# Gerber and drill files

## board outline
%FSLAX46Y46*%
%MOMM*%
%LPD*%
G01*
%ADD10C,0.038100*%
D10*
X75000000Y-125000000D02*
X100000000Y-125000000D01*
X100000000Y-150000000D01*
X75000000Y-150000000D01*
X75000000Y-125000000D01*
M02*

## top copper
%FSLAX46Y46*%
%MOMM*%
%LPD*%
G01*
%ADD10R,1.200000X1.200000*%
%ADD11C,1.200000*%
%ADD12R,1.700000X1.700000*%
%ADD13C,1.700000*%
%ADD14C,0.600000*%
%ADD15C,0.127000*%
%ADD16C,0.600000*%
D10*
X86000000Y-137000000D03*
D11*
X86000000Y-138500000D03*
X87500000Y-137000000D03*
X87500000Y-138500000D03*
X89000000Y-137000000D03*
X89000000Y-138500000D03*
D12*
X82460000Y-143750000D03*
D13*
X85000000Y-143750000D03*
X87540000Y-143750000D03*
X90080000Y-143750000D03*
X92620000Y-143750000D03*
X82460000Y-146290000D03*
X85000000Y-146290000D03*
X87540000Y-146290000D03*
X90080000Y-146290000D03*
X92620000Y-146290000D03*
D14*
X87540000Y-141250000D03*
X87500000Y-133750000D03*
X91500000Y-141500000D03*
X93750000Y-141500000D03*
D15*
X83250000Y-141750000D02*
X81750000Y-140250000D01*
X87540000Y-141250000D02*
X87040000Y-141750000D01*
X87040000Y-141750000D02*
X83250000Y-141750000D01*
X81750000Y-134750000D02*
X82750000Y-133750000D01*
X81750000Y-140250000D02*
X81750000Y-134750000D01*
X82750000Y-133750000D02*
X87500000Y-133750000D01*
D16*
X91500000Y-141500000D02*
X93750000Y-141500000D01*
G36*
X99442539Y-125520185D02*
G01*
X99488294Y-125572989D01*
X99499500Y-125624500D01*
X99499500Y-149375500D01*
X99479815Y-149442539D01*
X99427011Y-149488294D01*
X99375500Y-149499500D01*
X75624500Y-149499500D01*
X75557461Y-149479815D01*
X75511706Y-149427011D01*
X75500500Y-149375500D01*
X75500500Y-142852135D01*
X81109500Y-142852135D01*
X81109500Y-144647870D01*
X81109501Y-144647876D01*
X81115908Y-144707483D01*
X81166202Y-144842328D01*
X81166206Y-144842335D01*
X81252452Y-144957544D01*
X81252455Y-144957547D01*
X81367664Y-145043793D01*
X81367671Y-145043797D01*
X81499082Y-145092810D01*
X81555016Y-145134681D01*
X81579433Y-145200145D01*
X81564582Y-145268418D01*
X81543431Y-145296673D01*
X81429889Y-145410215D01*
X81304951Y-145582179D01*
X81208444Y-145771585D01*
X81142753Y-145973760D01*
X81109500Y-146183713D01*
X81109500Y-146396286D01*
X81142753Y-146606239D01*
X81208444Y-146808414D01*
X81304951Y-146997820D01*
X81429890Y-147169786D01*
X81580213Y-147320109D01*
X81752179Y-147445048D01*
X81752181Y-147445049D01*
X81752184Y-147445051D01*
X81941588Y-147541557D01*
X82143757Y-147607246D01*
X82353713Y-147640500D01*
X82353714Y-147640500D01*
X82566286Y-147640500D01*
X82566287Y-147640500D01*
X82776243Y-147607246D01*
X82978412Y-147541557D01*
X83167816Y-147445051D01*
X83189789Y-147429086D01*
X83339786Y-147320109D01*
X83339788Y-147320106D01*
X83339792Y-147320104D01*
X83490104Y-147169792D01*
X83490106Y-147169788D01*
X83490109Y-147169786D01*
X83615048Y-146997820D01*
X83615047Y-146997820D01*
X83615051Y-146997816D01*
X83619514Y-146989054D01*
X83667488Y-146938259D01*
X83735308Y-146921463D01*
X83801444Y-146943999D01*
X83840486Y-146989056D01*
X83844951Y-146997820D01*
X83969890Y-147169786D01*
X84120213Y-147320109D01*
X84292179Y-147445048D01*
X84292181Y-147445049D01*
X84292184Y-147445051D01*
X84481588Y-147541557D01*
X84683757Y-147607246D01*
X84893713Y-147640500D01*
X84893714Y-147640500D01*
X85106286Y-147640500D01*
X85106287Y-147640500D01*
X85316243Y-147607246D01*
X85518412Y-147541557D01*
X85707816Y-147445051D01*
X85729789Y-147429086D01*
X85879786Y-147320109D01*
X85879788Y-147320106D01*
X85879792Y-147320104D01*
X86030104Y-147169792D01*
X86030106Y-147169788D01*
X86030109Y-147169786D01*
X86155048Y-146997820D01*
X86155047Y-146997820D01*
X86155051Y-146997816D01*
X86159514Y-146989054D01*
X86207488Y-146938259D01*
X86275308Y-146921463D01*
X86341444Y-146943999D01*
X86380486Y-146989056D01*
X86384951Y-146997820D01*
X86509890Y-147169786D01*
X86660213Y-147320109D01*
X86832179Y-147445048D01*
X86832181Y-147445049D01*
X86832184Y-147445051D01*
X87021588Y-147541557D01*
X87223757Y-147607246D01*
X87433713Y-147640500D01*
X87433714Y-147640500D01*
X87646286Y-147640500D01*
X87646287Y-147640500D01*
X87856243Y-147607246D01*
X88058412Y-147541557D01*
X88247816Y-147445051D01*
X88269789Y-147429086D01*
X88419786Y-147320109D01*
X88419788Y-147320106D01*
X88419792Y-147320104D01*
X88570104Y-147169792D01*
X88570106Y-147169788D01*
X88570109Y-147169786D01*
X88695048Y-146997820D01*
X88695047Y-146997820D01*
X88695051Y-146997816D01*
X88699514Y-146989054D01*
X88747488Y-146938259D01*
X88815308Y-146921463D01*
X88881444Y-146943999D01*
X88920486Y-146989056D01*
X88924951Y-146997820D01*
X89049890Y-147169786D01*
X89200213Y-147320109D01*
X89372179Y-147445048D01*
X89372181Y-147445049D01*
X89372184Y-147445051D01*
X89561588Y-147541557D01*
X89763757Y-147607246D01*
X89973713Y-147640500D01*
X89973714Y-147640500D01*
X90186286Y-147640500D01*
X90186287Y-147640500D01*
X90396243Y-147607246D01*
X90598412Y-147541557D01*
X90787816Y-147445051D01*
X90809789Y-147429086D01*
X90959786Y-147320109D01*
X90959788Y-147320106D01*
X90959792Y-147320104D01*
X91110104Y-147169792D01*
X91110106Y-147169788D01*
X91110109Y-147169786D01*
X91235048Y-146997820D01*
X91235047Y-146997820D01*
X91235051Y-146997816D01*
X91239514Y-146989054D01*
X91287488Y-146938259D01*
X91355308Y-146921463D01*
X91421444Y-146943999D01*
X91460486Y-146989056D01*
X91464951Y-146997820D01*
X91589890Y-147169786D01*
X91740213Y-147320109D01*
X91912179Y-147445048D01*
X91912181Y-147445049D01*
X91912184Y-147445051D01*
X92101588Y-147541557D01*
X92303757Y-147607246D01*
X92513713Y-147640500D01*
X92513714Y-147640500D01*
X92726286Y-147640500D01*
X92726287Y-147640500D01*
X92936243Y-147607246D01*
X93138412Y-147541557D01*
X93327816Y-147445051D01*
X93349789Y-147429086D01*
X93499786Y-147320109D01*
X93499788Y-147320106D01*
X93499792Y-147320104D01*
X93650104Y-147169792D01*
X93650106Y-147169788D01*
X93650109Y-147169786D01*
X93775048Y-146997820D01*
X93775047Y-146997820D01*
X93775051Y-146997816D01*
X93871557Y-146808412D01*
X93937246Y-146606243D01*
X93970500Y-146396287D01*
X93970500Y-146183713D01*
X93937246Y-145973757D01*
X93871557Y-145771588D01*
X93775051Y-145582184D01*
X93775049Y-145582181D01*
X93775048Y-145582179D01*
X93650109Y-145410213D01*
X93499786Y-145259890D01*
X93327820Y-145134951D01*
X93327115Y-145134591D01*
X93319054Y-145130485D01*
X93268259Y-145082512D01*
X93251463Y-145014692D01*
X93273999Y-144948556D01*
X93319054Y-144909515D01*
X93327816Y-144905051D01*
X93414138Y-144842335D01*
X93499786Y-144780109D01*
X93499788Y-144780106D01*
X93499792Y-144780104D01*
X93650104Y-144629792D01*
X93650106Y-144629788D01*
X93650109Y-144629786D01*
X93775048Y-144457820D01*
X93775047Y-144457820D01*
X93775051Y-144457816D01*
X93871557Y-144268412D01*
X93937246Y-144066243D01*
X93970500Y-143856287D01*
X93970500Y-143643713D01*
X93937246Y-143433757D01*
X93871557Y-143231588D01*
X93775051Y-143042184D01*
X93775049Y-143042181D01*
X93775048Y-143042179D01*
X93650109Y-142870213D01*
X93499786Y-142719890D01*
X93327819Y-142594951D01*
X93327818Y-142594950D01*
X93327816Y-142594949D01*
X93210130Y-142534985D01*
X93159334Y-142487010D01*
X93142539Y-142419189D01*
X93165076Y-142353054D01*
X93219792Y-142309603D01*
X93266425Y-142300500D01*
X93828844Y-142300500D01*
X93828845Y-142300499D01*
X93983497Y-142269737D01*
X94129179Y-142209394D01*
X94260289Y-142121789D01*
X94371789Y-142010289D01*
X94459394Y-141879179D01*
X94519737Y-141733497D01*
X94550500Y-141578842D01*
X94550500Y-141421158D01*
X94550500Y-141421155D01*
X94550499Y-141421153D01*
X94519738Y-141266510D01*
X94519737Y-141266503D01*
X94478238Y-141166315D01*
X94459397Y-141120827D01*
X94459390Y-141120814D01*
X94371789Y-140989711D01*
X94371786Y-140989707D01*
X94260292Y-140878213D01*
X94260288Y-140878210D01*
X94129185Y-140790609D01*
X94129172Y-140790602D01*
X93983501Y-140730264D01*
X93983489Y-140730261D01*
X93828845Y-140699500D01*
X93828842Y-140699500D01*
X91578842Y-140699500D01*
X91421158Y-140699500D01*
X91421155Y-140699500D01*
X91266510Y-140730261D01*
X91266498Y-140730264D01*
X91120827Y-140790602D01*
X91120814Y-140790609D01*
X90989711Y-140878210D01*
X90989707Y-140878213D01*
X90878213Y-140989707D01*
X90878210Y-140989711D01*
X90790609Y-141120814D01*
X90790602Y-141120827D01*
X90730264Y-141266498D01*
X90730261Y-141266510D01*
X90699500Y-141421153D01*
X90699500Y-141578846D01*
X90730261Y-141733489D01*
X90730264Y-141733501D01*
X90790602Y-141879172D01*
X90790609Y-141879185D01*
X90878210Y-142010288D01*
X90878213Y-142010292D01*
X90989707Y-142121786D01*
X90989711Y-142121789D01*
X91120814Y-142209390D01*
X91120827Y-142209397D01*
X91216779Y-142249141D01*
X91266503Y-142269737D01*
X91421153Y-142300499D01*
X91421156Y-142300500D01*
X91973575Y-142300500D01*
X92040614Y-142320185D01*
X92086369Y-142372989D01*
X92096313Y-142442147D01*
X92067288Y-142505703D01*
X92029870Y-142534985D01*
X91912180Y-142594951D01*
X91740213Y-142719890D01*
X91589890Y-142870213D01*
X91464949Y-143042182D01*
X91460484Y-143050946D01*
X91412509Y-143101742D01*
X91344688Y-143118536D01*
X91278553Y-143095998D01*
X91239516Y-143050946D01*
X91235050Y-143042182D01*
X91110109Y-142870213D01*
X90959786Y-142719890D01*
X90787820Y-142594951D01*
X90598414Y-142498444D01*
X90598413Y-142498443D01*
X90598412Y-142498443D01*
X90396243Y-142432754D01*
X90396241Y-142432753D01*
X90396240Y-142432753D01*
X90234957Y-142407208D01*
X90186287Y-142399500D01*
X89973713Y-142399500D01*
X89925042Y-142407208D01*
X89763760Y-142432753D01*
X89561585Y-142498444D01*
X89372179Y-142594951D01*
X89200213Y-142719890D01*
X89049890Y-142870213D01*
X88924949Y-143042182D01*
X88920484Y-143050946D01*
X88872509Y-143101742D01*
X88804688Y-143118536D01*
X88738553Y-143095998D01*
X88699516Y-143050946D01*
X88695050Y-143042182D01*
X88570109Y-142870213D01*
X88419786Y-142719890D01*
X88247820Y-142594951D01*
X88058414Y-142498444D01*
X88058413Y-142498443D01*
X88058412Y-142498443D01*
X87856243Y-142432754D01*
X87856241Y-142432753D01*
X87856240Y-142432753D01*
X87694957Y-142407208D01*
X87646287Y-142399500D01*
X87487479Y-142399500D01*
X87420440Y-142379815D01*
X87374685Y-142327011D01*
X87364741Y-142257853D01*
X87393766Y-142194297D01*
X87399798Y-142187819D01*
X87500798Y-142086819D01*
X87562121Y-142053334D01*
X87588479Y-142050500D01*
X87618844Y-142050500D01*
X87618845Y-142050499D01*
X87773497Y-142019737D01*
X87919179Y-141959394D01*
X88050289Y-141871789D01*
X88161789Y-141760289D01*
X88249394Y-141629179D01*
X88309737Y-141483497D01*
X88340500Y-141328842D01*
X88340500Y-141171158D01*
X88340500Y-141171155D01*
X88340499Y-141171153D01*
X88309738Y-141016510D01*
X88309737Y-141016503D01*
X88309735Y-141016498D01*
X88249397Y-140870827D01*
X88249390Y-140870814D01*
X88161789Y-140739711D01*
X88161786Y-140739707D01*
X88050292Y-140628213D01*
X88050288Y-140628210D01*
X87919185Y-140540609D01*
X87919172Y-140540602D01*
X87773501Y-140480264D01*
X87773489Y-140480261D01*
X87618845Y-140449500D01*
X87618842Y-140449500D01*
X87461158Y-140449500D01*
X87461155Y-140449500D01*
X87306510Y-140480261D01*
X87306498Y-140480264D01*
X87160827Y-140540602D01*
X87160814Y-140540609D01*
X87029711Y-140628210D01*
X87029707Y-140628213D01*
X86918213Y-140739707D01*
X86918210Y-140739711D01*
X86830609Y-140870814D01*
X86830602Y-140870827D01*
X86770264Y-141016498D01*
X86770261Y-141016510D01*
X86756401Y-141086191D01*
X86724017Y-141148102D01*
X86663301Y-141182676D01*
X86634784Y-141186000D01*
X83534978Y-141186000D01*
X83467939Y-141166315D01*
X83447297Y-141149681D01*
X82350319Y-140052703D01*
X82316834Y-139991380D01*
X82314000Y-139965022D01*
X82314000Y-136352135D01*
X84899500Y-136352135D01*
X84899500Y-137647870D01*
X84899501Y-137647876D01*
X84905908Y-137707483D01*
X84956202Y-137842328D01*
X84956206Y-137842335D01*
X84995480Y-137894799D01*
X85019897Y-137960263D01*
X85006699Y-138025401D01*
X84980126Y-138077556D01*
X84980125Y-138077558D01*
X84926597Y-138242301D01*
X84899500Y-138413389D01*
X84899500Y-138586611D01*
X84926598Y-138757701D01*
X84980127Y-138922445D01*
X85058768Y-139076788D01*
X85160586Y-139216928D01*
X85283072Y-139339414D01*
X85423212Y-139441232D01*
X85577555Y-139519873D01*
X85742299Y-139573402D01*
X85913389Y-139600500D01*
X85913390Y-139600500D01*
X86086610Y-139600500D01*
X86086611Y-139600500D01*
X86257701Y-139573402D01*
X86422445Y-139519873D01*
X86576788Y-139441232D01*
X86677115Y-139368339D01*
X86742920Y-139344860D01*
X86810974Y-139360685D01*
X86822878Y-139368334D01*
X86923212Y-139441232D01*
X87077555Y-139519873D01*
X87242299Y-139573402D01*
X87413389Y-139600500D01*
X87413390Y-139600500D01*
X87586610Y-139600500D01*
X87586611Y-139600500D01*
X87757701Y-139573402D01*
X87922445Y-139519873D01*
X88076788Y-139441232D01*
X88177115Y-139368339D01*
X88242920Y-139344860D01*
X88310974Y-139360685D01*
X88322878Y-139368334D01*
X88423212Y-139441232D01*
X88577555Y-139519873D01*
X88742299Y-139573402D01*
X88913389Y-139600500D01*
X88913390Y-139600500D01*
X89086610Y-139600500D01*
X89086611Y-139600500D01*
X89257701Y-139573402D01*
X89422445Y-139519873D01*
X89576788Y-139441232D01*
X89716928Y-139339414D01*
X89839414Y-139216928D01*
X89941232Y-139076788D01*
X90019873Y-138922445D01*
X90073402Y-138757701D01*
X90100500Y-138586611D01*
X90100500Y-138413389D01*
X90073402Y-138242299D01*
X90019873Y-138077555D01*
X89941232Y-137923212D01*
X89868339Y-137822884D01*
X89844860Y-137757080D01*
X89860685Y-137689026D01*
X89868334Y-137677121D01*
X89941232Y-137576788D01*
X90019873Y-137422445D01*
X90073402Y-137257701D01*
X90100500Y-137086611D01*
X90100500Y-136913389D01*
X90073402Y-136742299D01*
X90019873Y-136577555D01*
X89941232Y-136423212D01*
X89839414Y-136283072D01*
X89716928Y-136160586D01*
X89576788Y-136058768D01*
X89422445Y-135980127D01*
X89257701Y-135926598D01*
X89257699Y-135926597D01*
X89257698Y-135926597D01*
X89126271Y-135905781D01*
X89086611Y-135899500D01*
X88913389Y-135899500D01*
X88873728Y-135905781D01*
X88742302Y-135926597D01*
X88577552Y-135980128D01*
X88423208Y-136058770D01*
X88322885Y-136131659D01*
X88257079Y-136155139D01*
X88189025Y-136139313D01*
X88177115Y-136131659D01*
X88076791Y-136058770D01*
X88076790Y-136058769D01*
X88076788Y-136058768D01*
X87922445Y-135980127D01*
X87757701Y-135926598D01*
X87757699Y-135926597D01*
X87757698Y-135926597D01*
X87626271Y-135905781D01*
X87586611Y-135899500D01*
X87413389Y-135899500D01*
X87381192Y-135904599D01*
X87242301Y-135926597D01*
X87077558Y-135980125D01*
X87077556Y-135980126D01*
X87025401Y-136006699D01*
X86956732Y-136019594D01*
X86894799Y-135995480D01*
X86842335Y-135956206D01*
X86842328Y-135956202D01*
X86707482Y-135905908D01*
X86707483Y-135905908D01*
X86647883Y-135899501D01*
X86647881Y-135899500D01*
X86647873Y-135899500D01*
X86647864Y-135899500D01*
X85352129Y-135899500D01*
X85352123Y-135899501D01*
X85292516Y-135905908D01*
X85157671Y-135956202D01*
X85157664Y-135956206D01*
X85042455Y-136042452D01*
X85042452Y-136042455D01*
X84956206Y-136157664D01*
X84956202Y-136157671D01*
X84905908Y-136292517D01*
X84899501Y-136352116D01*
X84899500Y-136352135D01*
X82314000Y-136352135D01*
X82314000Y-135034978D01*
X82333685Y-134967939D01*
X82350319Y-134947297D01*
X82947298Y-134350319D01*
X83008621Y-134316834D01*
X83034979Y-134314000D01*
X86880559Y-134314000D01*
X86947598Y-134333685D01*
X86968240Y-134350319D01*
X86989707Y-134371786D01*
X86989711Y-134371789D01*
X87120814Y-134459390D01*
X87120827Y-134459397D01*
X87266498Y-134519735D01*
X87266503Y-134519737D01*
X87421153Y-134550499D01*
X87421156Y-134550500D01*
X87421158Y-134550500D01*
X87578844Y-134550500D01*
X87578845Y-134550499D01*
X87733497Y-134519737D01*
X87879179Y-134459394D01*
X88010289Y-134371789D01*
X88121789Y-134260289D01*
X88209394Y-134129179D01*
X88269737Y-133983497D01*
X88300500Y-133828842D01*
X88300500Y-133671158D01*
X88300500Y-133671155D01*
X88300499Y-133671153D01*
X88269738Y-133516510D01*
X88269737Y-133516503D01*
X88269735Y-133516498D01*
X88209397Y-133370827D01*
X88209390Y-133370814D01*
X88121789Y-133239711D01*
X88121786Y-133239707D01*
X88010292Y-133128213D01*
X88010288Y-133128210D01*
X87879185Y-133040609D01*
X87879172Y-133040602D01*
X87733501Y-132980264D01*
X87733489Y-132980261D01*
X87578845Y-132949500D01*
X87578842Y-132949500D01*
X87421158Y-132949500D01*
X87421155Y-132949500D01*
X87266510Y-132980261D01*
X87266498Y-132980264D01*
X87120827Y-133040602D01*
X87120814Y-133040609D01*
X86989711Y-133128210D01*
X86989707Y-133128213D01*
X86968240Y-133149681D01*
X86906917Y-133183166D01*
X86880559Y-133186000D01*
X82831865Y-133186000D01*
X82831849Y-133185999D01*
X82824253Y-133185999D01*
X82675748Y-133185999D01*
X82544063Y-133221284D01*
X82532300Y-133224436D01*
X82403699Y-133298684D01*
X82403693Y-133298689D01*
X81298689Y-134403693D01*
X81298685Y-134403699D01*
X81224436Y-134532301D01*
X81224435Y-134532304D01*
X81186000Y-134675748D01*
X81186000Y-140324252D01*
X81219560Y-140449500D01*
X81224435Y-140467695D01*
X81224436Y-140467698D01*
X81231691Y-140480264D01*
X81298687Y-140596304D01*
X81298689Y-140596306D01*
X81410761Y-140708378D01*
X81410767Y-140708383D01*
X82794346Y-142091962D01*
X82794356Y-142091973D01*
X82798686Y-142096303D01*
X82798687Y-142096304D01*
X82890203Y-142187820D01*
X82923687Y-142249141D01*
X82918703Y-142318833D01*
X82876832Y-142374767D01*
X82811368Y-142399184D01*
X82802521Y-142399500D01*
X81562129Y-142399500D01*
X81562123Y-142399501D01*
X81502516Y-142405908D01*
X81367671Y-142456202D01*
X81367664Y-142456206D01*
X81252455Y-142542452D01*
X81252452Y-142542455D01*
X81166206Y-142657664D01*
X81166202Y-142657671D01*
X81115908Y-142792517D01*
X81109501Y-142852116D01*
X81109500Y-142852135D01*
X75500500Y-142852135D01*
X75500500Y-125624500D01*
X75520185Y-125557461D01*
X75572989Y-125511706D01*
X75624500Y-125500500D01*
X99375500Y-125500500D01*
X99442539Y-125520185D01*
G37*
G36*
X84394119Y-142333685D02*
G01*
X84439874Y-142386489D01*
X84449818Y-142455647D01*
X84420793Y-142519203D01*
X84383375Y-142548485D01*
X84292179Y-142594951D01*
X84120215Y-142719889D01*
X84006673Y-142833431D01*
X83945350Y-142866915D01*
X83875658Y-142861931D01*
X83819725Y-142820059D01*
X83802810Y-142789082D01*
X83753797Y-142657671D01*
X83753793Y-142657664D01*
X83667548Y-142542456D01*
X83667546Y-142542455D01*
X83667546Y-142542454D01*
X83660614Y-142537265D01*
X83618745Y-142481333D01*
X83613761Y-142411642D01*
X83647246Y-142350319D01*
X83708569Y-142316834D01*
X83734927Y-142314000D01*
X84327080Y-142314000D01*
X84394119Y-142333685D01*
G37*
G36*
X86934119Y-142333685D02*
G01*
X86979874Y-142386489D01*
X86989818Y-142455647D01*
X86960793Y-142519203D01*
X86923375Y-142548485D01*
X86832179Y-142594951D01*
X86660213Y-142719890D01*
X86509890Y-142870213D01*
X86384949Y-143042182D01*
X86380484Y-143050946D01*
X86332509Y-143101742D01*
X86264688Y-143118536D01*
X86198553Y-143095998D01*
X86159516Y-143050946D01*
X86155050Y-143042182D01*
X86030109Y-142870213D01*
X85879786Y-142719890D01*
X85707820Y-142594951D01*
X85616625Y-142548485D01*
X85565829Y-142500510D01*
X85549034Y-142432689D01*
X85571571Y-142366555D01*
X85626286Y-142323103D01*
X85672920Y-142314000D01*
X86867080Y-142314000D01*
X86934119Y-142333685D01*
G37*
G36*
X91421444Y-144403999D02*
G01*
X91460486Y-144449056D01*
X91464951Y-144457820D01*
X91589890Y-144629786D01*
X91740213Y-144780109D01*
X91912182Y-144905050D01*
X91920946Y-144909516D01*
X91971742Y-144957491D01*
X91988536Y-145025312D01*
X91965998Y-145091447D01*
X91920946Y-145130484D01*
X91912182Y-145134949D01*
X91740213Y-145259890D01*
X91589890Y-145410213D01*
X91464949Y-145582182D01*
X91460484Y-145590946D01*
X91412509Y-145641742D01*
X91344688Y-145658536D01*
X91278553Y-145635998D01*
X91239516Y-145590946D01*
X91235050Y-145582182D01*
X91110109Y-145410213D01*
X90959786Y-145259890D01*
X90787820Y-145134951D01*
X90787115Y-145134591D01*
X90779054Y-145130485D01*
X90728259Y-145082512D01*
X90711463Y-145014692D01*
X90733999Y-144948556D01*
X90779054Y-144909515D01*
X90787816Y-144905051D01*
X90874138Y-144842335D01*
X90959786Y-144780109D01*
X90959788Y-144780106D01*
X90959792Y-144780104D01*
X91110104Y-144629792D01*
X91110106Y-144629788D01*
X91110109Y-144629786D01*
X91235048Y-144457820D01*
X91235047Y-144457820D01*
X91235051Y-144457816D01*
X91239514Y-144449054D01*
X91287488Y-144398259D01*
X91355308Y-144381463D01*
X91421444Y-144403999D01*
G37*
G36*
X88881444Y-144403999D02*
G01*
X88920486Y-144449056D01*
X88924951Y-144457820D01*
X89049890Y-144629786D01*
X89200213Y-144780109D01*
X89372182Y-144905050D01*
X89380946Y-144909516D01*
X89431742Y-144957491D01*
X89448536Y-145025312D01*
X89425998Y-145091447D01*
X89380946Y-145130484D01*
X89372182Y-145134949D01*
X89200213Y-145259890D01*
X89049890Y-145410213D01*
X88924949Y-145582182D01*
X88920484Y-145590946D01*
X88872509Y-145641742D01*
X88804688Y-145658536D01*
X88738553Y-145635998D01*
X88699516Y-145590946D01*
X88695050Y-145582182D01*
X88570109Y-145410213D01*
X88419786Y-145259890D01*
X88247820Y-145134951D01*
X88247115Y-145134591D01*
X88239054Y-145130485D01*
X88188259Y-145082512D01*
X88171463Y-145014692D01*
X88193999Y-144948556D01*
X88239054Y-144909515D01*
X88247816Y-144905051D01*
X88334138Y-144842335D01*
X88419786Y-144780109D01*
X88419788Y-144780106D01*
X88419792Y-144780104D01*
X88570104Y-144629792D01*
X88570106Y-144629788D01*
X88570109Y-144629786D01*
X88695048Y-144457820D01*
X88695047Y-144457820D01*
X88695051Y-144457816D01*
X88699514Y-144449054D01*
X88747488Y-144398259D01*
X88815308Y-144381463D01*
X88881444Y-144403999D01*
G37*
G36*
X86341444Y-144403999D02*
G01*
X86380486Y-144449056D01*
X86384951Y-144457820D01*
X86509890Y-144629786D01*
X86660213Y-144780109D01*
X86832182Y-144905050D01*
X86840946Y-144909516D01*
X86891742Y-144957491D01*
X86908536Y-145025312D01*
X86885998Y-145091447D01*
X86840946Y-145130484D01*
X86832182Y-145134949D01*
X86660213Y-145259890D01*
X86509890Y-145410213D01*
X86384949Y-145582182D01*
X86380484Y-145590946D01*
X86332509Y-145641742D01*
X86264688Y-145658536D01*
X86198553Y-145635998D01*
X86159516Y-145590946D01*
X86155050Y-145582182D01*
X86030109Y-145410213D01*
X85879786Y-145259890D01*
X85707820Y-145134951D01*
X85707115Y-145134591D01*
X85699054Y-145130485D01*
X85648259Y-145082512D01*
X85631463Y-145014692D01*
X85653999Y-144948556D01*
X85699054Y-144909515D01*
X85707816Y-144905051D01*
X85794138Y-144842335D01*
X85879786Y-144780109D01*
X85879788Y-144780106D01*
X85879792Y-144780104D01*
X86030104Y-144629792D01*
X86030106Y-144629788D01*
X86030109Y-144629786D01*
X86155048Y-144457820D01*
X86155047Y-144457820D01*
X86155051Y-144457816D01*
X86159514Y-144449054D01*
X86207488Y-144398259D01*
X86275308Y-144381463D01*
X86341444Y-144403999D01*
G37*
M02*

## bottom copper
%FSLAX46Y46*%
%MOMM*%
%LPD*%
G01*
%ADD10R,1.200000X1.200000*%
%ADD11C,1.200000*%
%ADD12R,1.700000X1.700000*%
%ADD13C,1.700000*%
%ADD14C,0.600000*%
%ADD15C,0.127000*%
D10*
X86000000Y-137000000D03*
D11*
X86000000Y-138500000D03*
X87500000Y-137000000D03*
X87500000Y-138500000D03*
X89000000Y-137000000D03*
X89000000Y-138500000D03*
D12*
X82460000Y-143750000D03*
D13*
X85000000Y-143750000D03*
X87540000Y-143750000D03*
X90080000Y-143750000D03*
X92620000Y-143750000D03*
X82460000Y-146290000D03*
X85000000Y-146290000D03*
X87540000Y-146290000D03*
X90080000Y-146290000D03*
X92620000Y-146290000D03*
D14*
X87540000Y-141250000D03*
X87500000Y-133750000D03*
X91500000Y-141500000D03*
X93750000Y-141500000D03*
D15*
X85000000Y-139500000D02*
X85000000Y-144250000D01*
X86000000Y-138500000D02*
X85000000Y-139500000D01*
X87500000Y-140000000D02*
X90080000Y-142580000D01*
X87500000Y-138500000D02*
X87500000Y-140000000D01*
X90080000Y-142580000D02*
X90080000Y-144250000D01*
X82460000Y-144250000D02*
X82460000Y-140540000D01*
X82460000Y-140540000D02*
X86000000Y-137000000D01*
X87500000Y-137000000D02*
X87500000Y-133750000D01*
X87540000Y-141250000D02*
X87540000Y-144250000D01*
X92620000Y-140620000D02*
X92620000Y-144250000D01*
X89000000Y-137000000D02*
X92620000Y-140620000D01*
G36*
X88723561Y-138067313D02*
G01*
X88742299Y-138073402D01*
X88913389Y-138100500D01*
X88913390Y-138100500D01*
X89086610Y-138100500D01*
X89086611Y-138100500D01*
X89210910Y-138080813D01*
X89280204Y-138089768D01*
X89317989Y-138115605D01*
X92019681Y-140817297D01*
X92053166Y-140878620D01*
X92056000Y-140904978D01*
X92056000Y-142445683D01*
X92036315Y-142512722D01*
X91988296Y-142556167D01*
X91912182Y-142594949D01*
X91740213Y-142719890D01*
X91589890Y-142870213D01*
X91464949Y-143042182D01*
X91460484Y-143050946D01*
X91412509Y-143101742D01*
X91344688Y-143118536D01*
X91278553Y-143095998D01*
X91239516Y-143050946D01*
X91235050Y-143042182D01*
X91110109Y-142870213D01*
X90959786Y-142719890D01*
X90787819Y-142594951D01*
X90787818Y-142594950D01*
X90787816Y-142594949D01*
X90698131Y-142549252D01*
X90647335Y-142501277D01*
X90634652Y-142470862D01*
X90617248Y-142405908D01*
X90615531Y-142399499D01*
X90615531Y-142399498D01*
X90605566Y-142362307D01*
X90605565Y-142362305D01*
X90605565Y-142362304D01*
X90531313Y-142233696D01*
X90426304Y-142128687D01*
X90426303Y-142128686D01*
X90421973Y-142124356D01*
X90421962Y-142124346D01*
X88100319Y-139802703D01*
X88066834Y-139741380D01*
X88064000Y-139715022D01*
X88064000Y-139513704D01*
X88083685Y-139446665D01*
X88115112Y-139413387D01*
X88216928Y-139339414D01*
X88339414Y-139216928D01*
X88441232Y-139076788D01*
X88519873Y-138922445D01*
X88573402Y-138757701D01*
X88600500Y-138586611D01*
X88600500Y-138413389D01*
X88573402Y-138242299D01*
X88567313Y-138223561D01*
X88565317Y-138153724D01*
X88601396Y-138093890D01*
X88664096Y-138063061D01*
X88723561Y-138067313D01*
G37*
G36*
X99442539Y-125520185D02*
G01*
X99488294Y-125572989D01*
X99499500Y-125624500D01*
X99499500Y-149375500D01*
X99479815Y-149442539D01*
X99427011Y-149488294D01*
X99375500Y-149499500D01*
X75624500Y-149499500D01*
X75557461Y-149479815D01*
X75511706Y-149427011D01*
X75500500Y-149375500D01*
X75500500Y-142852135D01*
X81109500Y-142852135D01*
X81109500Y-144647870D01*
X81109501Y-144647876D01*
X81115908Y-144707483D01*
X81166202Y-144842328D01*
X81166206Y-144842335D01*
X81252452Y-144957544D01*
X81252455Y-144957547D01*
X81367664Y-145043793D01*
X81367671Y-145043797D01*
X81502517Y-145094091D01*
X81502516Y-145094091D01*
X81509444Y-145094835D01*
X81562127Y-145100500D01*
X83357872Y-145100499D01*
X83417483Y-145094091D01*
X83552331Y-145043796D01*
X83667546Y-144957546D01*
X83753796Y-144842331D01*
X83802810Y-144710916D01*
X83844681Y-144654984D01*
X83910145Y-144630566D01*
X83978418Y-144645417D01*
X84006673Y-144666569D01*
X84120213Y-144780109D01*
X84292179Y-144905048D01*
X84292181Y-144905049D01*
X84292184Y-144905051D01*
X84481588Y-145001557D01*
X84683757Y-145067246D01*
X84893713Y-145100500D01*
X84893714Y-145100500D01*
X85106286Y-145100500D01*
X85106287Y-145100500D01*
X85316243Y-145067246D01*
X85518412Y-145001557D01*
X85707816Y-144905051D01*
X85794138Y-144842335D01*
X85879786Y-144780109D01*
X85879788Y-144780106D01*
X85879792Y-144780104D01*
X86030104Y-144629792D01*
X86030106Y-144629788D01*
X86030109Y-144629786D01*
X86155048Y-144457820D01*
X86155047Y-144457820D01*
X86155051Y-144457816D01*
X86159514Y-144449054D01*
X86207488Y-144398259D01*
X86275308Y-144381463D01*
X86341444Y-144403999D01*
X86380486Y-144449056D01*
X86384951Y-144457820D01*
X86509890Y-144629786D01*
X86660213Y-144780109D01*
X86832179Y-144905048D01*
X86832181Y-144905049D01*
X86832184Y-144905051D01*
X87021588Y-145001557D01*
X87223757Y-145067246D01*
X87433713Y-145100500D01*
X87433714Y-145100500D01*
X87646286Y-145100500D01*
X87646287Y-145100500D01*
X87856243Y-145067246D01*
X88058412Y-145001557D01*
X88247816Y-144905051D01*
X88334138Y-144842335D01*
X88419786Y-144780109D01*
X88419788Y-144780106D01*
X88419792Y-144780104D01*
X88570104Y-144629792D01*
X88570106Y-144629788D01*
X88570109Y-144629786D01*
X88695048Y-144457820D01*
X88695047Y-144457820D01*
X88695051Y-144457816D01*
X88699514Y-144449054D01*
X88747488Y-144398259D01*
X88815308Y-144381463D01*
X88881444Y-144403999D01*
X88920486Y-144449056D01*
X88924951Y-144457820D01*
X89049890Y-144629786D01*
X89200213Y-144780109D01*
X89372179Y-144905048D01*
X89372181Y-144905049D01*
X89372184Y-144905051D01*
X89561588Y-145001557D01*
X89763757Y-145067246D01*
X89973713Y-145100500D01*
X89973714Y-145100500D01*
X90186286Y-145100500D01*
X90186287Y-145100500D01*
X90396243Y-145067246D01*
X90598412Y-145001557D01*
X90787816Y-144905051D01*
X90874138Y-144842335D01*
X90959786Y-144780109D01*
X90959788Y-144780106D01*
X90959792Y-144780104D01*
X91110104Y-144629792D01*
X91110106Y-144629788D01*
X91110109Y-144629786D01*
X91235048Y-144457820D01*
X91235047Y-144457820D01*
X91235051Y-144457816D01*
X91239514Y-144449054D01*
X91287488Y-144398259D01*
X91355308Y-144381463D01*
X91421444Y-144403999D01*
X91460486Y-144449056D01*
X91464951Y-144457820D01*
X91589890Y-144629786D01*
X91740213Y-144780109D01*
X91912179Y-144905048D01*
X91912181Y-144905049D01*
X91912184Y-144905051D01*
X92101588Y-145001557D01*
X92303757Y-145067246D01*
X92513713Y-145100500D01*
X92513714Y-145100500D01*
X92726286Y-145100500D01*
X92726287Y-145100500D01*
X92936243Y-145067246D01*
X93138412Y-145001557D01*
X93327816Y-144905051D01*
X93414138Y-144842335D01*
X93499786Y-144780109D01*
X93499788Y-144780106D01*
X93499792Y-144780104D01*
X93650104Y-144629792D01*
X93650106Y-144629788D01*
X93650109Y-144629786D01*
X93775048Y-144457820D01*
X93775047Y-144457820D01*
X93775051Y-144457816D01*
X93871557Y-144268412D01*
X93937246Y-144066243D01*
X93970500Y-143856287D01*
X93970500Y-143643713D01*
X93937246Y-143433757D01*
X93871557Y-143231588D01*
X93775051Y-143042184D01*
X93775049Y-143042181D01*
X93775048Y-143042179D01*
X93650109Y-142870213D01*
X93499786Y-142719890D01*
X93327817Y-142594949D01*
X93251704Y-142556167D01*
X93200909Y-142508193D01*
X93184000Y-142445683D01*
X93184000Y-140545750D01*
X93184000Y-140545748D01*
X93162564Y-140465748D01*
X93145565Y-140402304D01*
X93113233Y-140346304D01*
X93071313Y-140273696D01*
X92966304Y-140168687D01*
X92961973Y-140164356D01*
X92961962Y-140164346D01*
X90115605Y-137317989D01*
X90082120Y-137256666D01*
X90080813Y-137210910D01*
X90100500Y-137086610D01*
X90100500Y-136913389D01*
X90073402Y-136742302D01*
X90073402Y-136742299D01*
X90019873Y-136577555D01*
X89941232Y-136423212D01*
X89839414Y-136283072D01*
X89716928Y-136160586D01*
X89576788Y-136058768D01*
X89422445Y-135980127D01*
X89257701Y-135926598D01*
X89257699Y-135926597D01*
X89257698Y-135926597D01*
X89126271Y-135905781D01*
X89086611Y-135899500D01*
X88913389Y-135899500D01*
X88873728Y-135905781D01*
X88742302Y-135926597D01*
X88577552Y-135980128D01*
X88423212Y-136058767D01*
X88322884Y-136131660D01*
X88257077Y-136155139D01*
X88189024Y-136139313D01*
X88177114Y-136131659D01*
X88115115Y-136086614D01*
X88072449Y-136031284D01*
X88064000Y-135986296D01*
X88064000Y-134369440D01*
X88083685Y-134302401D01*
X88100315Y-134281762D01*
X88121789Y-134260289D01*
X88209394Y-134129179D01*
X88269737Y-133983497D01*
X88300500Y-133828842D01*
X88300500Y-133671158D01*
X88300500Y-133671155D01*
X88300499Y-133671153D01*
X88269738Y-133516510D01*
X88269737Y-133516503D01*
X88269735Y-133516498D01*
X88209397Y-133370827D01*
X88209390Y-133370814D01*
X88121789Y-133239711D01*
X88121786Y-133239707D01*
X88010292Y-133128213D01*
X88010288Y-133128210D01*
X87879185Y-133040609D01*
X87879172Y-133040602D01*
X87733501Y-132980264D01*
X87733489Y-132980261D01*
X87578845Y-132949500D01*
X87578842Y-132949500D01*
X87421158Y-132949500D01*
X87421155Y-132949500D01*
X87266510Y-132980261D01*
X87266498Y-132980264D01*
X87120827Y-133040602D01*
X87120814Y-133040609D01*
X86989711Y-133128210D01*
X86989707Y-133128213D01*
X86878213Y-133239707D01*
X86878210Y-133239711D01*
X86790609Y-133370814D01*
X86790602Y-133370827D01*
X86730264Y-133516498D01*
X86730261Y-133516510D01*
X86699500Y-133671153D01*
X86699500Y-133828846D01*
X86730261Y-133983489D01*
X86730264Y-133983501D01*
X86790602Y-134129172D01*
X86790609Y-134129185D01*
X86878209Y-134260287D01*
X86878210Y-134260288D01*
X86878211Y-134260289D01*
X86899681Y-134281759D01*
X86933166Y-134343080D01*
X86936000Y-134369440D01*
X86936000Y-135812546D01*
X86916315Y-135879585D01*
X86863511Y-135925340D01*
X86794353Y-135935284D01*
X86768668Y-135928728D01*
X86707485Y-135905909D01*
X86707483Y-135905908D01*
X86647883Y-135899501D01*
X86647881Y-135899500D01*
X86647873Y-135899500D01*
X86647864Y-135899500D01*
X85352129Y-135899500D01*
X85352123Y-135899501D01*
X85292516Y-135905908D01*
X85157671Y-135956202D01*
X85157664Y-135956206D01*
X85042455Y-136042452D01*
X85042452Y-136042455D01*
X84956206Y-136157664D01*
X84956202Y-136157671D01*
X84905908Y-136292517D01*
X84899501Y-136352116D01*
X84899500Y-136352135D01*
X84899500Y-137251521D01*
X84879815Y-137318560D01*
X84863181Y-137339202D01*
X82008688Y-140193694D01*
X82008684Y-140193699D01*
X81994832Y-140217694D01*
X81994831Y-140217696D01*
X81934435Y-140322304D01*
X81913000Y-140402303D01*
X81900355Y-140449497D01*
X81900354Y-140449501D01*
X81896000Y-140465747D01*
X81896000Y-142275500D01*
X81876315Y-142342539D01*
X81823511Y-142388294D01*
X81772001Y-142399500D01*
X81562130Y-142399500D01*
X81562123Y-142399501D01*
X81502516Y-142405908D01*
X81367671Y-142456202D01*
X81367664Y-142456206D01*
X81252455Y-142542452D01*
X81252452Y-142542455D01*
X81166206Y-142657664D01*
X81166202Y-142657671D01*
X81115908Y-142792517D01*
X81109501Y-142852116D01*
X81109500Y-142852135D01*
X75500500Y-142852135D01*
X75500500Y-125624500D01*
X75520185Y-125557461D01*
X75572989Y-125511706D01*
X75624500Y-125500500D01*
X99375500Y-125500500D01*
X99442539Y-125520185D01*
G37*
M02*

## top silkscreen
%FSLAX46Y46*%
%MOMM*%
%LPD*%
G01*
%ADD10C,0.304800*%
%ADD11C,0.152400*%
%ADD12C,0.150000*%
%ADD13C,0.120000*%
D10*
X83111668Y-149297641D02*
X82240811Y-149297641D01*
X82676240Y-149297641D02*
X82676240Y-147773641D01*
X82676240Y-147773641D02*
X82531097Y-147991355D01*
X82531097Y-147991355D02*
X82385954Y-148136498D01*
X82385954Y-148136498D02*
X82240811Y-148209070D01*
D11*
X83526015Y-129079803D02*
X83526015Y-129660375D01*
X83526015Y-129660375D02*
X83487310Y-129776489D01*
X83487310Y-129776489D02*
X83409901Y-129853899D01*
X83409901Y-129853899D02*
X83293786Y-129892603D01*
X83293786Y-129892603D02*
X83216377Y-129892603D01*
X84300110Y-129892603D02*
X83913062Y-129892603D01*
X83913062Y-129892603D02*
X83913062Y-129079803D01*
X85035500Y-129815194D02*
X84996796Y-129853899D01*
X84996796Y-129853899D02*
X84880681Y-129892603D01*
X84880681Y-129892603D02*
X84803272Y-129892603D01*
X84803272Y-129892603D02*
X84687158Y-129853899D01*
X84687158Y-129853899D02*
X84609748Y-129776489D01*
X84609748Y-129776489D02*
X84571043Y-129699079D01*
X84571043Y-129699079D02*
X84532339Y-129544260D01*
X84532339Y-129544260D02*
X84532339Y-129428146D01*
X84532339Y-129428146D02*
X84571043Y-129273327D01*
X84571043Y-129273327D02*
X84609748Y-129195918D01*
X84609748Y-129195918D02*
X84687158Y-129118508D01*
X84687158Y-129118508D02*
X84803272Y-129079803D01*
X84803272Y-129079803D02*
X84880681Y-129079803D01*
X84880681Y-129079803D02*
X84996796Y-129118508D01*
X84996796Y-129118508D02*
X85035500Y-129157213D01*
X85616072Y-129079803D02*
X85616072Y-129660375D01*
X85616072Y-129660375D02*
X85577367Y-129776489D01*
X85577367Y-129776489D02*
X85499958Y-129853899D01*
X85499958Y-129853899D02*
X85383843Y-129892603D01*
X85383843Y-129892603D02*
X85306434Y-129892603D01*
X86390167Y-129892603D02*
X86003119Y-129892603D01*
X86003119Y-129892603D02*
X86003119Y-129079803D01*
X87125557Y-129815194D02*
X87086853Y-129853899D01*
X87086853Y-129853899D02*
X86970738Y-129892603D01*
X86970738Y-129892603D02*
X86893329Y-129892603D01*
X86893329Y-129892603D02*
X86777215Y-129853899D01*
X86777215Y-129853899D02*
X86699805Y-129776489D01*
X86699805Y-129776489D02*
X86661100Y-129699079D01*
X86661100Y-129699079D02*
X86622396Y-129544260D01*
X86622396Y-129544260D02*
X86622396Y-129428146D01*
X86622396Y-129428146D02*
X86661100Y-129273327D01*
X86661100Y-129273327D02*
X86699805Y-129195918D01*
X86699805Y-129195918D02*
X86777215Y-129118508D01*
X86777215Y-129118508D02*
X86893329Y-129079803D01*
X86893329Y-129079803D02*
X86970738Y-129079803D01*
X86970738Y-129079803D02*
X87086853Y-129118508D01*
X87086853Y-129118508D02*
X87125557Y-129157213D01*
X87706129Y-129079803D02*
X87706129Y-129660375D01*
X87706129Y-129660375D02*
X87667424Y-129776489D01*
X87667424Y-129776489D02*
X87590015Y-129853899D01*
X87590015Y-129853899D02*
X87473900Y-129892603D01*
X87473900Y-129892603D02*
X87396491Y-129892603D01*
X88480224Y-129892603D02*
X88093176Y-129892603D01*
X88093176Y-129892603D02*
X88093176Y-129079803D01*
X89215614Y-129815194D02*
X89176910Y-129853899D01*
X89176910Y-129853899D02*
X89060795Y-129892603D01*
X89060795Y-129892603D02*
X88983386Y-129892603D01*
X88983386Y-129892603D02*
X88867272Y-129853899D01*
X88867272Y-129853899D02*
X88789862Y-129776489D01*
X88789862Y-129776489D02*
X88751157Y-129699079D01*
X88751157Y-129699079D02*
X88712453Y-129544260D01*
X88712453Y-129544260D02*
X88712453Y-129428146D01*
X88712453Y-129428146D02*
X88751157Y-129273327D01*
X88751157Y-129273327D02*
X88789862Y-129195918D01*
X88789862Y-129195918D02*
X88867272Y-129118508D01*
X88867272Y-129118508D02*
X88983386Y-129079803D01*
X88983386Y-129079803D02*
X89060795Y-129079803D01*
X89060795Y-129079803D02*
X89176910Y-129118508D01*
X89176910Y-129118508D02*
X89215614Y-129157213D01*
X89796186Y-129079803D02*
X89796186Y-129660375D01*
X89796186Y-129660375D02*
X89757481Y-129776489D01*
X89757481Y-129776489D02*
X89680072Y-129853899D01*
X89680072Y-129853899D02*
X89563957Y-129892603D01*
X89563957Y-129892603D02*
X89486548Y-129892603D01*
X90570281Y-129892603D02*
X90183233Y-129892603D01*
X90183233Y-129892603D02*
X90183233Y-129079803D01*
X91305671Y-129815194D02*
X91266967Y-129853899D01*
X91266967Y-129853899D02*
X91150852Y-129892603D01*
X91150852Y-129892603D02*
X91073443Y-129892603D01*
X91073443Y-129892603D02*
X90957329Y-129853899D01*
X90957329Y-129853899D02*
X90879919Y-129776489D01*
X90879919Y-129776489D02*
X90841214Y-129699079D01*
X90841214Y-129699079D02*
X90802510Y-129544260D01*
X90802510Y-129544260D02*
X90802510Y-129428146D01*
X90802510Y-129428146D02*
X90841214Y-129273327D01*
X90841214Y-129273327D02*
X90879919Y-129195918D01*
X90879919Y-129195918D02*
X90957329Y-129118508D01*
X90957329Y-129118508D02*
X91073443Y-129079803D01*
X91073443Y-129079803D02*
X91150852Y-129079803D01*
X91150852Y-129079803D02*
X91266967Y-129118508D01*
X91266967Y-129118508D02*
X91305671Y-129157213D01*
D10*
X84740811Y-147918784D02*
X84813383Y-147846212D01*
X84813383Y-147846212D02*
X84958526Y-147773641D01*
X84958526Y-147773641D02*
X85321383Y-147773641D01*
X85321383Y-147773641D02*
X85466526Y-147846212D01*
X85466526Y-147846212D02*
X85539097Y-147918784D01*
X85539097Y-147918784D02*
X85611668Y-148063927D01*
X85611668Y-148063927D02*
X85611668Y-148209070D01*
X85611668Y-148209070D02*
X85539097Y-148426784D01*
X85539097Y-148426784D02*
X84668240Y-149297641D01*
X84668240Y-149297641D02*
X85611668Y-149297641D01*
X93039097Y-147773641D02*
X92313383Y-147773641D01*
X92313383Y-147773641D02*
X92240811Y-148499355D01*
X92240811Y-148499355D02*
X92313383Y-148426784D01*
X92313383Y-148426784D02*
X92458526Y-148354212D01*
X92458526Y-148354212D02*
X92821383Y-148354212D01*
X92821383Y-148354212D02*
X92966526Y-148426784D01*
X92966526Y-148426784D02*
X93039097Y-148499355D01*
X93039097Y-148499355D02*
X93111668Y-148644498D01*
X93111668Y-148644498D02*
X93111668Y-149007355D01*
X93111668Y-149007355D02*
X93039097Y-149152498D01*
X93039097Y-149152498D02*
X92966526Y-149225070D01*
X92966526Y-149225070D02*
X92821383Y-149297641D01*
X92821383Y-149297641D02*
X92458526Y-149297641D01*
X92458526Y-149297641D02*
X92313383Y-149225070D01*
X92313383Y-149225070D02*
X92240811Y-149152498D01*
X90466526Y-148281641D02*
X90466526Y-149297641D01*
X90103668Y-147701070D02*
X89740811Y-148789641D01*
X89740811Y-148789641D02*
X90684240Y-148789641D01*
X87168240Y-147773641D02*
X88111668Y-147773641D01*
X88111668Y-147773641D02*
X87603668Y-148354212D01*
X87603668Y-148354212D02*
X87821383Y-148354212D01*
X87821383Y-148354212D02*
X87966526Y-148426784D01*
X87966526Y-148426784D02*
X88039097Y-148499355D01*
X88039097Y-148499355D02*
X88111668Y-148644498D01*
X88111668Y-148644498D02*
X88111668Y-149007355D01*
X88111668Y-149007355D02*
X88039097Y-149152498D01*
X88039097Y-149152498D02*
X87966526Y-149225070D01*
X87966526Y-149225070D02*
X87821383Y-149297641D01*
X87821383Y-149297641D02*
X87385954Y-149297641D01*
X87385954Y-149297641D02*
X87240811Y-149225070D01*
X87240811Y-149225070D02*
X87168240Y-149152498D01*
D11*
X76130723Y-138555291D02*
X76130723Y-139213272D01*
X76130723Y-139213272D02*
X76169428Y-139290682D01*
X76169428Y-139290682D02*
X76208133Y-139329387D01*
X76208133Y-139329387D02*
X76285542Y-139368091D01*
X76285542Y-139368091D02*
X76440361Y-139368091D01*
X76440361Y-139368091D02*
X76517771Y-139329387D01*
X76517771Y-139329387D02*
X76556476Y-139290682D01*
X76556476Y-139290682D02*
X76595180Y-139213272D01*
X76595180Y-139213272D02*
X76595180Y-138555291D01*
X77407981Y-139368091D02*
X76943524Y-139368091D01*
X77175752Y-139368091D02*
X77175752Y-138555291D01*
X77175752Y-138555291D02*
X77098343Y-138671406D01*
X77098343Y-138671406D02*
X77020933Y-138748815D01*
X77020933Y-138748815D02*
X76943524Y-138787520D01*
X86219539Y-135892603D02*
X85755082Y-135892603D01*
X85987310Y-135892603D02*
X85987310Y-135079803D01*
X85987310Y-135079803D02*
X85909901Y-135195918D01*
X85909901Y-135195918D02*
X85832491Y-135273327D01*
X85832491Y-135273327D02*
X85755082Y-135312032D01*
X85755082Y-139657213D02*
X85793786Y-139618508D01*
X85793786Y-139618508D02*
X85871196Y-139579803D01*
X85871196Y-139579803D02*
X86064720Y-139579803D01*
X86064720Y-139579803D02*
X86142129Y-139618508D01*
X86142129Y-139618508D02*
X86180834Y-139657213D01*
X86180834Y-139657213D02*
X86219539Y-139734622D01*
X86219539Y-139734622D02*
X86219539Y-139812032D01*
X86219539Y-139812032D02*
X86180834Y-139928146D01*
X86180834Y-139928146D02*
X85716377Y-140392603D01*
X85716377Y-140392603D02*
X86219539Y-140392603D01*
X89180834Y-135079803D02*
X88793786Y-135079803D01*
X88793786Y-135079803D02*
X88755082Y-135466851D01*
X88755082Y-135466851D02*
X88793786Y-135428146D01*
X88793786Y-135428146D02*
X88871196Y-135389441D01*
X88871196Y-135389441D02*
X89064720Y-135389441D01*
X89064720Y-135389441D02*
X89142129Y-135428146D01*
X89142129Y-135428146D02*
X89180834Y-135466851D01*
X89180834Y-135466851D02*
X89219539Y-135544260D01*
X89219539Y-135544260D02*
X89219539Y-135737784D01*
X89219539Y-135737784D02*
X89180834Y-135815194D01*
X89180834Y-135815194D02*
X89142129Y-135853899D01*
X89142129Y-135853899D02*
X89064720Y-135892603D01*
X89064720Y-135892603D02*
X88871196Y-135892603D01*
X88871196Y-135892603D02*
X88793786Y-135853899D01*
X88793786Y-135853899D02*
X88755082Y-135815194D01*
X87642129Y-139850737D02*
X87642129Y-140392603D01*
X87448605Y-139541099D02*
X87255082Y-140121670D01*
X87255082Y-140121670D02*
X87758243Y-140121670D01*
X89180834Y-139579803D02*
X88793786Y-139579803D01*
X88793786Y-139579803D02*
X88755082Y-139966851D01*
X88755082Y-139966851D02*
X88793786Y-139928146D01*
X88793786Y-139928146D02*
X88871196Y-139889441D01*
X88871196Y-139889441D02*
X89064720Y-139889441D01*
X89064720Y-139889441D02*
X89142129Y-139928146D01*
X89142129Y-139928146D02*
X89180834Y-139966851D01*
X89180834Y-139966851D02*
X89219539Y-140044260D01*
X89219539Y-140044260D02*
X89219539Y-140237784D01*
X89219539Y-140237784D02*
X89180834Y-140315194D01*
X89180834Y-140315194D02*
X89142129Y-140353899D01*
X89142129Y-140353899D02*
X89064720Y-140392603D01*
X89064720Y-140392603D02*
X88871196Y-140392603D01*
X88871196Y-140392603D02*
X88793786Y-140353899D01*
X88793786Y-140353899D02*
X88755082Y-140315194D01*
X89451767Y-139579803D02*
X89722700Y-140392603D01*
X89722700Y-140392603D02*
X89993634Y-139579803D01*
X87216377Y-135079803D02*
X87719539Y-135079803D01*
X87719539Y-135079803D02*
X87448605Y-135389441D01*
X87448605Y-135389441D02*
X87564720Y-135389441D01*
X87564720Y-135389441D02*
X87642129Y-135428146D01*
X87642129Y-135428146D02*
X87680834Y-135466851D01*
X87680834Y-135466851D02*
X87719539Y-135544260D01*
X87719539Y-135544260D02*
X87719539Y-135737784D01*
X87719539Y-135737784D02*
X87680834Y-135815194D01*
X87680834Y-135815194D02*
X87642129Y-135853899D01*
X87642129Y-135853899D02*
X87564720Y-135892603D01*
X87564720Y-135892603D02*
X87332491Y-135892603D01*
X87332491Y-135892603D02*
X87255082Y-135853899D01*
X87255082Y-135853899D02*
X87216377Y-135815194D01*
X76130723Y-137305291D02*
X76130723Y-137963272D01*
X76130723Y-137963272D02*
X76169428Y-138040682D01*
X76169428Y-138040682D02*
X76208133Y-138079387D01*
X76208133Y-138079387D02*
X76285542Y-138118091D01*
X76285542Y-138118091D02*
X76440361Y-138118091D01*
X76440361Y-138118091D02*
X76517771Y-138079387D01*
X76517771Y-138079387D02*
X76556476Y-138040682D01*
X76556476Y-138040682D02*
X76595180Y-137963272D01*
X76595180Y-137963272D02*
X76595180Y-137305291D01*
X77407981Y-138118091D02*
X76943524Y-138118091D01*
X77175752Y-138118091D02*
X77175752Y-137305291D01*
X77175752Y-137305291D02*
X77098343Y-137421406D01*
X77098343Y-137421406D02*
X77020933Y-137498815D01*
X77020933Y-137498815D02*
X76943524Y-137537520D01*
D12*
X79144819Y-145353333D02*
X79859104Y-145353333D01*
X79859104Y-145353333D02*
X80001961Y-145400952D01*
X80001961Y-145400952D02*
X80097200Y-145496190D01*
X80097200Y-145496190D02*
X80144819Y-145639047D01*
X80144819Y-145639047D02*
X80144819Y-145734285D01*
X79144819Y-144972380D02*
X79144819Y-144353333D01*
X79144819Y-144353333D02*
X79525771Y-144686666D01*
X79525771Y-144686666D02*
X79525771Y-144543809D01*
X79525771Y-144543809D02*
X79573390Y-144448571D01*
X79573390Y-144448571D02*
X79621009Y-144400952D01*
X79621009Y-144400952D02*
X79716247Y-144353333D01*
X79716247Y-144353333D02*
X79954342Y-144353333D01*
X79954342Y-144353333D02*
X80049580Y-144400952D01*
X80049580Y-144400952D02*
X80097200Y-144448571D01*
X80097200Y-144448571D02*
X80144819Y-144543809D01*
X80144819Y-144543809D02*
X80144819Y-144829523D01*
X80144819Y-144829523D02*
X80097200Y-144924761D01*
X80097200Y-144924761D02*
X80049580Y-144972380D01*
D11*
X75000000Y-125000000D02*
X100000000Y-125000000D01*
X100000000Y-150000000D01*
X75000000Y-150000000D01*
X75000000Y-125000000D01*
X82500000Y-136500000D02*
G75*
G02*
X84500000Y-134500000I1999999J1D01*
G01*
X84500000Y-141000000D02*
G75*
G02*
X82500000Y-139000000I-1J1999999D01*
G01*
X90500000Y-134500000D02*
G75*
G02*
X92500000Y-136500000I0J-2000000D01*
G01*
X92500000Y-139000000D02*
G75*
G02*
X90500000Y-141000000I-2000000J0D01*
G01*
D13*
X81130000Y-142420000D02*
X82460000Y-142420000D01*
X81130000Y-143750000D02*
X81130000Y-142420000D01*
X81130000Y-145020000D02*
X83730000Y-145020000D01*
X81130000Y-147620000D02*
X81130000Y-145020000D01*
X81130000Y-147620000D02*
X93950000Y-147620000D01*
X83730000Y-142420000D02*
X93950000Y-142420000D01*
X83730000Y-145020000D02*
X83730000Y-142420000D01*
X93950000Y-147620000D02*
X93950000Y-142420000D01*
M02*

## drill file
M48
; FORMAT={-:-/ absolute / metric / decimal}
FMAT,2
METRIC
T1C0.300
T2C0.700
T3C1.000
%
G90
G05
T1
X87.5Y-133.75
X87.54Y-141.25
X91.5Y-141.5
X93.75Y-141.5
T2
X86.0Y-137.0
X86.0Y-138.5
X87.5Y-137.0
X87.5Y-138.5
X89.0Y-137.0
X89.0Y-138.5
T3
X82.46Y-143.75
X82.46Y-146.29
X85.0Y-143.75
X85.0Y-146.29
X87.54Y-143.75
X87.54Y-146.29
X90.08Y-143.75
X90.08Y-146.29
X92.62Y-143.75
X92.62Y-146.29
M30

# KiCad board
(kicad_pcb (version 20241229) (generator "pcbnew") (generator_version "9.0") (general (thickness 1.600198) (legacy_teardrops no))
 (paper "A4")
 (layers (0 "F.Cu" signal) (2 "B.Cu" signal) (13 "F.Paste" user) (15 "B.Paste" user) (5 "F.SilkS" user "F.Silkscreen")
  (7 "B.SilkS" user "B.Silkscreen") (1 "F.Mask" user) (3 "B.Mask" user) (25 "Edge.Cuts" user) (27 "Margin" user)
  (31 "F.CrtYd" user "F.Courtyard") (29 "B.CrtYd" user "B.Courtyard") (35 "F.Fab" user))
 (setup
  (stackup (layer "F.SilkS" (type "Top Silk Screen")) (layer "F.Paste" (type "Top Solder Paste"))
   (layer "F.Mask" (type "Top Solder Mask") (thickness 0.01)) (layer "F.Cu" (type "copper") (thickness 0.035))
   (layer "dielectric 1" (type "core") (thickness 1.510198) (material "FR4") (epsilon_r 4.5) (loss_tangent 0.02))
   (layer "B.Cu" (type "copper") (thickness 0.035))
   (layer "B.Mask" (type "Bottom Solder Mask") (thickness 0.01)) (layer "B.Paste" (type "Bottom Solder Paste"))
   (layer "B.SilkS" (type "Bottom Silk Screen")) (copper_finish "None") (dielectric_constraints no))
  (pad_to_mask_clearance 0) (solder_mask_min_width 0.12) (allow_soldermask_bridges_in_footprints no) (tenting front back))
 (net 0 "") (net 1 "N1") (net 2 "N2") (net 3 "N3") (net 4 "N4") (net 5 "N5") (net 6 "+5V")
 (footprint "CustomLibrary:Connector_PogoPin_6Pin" (layer "F.Cu") (at 87.5 138)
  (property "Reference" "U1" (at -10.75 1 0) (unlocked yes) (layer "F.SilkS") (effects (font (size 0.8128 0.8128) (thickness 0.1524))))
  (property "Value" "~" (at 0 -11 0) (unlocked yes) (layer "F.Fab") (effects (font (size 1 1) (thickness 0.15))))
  (fp_rect (start -12.5 -13) (end 12.5 12) (stroke (width 0.1524) (type default)) (fill no) (layer "F.SilkS"))
  (fp_arc (start -5 -1.5) (mid -4.414214 -2.914214) (end -3 -3.5) (stroke (width 0.1524) (type default)) (layer "F.SilkS"))
  (fp_arc (start -3 3) (mid -4.414214 2.414214) (end -5 1) (stroke (width 0.1524) (type default)) (layer "F.SilkS"))
  (fp_arc (start 3 -3.5) (mid 4.414214 -2.914214) (end 5 -1.5) (stroke (width 0.1524) (type default)) (layer "F.SilkS"))
  (fp_arc (start 5 1) (mid 4.414214 2.414214) (end 3 3) (stroke (width 0.1524) (type default)) (layer "F.SilkS"))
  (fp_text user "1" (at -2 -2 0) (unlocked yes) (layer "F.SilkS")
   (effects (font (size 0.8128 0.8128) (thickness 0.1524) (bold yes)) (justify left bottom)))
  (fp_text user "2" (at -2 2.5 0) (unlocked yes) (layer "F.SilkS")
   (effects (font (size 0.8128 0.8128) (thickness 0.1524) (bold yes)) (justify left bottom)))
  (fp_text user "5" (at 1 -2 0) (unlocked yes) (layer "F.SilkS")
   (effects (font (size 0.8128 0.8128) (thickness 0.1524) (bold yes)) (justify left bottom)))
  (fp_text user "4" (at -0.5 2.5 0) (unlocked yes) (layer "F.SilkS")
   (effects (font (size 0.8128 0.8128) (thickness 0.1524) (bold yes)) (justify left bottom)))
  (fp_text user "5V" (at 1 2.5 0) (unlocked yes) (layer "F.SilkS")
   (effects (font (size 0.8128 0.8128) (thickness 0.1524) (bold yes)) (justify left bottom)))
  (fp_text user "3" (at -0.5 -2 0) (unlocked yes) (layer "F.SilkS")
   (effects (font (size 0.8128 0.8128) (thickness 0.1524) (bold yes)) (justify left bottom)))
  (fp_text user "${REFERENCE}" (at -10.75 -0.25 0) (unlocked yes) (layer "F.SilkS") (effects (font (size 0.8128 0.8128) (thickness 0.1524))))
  (pad "1" thru_hole rect (at -1.5 -1) (size 1.2 1.2) (drill 0.7) (layers "*.Cu" "*.Mask") (remove_unused_layers no) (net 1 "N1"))
  (pad "2" thru_hole circle (at -1.5 0.5) (size 1.2 1.2) (drill 0.7) (layers "*.Cu" "*.Mask") (remove_unused_layers no) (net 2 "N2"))
  (pad "3" thru_hole circle (at 0 -1) (size 1.2 1.2) (drill 0.7) (layers "*.Cu" "*.Mask") (remove_unused_layers no) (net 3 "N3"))
  (pad "4" thru_hole circle (at 0 0.5) (size 1.2 1.2) (drill 0.7) (layers "*.Cu" "*.Mask") (remove_unused_layers no) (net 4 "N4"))
  (pad "5" thru_hole circle (at 1.5 -1) (size 1.2 1.2) (drill 0.7) (layers "*.Cu" "*.Mask") (remove_unused_layers no) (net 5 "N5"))
  (pad "6" thru_hole circle (at 1.5 0.5) (size 1.2 1.2) (drill 0.7) (layers "*.Cu" "*.Mask") (remove_unused_layers no) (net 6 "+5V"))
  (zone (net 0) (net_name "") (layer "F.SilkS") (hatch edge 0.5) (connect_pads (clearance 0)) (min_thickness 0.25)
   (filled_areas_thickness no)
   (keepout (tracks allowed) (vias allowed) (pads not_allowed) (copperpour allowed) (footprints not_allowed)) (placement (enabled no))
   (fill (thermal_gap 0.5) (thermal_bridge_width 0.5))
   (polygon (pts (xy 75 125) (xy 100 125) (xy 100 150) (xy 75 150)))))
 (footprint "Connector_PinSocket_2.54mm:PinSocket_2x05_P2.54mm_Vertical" (layer "F.Cu") (at 82.46 143.75 90)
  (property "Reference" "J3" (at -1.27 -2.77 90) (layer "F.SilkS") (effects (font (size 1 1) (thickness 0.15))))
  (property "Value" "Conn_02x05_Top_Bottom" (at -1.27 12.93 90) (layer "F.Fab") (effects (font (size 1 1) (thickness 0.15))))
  (fp_line (start 1.33 -1.33) (end 1.33 0) (stroke (width 0.12) (type solid)) (layer "F.SilkS"))
  (fp_line (start 0 -1.33) (end 1.33 -1.33) (stroke (width 0.12) (type solid)) (layer "F.SilkS"))
  (fp_line (start -1.27 -1.33) (end -1.27 1.27) (stroke (width 0.12) (type solid)) (layer "F.SilkS"))
  (fp_line (start -3.87 -1.33) (end -1.27 -1.33) (stroke (width 0.12) (type solid)) (layer "F.SilkS"))
  (fp_line (start -3.87 -1.33) (end -3.87 11.49) (stroke (width 0.12) (type solid)) (layer "F.SilkS"))
  (fp_line (start 1.33 1.27) (end 1.33 11.49) (stroke (width 0.12) (type solid)) (layer "F.SilkS"))
  (fp_line (start -1.27 1.27) (end 1.33 1.27) (stroke (width 0.12) (type solid)) (layer "F.SilkS"))
  (fp_line (start -3.87 11.49) (end 1.33 11.49) (stroke (width 0.12) (type solid)) (layer "F.SilkS"))
  (pad "1" thru_hole rect (at 0 0 90) (size 1.7 1.7) (drill 1) (layers "*.Cu" "*.Mask") (remove_unused_layers no) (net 1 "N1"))
  (pad "2" thru_hole circle (at 0 2.54 90) (size 1.7 1.7) (drill 1) (layers "*.Cu" "*.Mask") (remove_unused_layers no) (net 2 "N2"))
  (pad "3" thru_hole circle (at 0 5.08 90) (size 1.7 1.7) (drill 1) (layers "*.Cu" "*.Mask") (remove_unused_layers no) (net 3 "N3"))
  (pad "4" thru_hole circle (at 0 7.62 90) (size 1.7 1.7) (drill 1) (layers "*.Cu" "*.Mask" "B.Adhes") (remove_unused_layers no)
   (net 4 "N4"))
  (pad "5" thru_hole circle (at 0 10.16 90) (size 1.7 1.7) (drill 1) (layers "*.Cu" "*.Mask") (remove_unused_layers no) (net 5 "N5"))
  (pad "6" thru_hole circle (at -2.54 0 90) (size 1.7 1.7) (drill 1) (layers "*.Cu" "*.Mask") (remove_unused_layers no) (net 6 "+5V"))
  (pad "7" thru_hole circle (at -2.54 2.54 90) (size 1.7 1.7) (drill 1) (layers "*.Cu" "*.Mask") (remove_unused_layers no) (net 6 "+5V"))
  (pad "8" thru_hole circle (at -2.54 5.08 90) (size 1.7 1.7) (drill 1) (layers "*.Cu" "*.Mask") (remove_unused_layers no) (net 6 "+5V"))
  (pad "9" thru_hole circle (at -2.54 7.62 90) (size 1.7 1.7) (drill 1) (layers "*.Cu" "*.Mask") (remove_unused_layers no) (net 6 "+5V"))
  (pad "10" thru_hole circle (at -2.54 10.16 90) (size 1.7 1.7) (drill 1) (layers "*.Cu" "*.Mask") (remove_unused_layers no) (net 6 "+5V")))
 (gr_rect (start 75 125) (end 100 150) (stroke (width 0.0381) (type solid)) (fill no) (layer "Edge.Cuts"))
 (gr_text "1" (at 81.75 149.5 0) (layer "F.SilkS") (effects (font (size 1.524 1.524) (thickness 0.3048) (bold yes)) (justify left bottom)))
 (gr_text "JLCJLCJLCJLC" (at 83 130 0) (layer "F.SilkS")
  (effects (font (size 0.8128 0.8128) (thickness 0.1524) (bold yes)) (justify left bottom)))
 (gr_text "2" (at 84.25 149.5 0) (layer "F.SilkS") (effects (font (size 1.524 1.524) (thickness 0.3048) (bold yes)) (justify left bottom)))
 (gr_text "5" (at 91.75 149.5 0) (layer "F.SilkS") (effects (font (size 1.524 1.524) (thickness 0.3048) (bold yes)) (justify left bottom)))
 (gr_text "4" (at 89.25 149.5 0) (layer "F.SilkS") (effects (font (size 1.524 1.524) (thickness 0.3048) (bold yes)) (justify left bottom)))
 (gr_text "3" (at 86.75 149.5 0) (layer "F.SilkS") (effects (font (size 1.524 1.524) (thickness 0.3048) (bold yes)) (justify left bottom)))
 (segment (start 85 139.5) (end 85 144.25) (width 0.127) (layer "B.Cu") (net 2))
 (segment (start 86 138.5) (end 85 139.5) (width 0.127) (layer "B.Cu") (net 2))
 (segment (start 87.5 140) (end 90.08 142.58) (width 0.127) (layer "B.Cu") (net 4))
 (segment (start 87.5 138.5) (end 87.5 140) (width 0.127) (layer "B.Cu") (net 4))
 (segment (start 90.08 142.58) (end 90.08 144.25) (width 0.127) (layer "B.Cu") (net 4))
 (segment (start 82.46 144.25) (end 82.46 140.54) (width 0.127) (layer "B.Cu") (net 1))
 (segment (start 82.46 140.54) (end 86 137) (width 0.127) (layer "B.Cu") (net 1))
 (segment (start 83.25 141.75) (end 81.75 140.25) (width 0.127) (layer "F.Cu") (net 3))
 (segment (start 87.54 141.25) (end 87.04 141.75) (width 0.127) (layer "F.Cu") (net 3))
 (segment (start 87.04 141.75) (end 83.25 141.75) (width 0.127) (layer "F.Cu") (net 3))
 (segment (start 81.75 134.75) (end 82.75 133.75) (width 0.127) (layer "F.Cu") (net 3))
 (segment (start 81.75 140.25) (end 81.75 134.75) (width 0.127) (layer "F.Cu") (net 3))
 (segment (start 82.75 133.75) (end 87.5 133.75) (width 0.127) (layer "F.Cu") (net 3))
 (via (at 87.54 141.25) (size 0.6) (drill 0.3) (layers "F.Cu" "B.Cu") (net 3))
 (via (at 87.5 133.75) (size 0.6) (drill 0.3) (layers "F.Cu" "B.Cu") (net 3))
 (segment (start 87.5 137) (end 87.5 133.75) (width 0.127) (layer "B.Cu") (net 3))
 (segment (start 87.54 141.25) (end 87.54 144.25) (width 0.127) (layer "B.Cu") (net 3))
 (segment (start 92.62 140.62) (end 92.62 144.25) (width 0.127) (layer "B.Cu") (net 5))
 (segment (start 89 137) (end 92.62 140.62) (width 0.127) (layer "B.Cu") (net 5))
 (segment (start 91.5 141.5) (end 93.75 141.5) (width 0.6) (layer "F.Cu") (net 6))
 (via (at 91.5 141.5) (size 0.6) (drill 0.3) (layers "F.Cu" "B.Cu") (free yes) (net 6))
 (via (at 93.75 141.5) (size 0.6) (drill 0.3) (layers "F.Cu" "B.Cu") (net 6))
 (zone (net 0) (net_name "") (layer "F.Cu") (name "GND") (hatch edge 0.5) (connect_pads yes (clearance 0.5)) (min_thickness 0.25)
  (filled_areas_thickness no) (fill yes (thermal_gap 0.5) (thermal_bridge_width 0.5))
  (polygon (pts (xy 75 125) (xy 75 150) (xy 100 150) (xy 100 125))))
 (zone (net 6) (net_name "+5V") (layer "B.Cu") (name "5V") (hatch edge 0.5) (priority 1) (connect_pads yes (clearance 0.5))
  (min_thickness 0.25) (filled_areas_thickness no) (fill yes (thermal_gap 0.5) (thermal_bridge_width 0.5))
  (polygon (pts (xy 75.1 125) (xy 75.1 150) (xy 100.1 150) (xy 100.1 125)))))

